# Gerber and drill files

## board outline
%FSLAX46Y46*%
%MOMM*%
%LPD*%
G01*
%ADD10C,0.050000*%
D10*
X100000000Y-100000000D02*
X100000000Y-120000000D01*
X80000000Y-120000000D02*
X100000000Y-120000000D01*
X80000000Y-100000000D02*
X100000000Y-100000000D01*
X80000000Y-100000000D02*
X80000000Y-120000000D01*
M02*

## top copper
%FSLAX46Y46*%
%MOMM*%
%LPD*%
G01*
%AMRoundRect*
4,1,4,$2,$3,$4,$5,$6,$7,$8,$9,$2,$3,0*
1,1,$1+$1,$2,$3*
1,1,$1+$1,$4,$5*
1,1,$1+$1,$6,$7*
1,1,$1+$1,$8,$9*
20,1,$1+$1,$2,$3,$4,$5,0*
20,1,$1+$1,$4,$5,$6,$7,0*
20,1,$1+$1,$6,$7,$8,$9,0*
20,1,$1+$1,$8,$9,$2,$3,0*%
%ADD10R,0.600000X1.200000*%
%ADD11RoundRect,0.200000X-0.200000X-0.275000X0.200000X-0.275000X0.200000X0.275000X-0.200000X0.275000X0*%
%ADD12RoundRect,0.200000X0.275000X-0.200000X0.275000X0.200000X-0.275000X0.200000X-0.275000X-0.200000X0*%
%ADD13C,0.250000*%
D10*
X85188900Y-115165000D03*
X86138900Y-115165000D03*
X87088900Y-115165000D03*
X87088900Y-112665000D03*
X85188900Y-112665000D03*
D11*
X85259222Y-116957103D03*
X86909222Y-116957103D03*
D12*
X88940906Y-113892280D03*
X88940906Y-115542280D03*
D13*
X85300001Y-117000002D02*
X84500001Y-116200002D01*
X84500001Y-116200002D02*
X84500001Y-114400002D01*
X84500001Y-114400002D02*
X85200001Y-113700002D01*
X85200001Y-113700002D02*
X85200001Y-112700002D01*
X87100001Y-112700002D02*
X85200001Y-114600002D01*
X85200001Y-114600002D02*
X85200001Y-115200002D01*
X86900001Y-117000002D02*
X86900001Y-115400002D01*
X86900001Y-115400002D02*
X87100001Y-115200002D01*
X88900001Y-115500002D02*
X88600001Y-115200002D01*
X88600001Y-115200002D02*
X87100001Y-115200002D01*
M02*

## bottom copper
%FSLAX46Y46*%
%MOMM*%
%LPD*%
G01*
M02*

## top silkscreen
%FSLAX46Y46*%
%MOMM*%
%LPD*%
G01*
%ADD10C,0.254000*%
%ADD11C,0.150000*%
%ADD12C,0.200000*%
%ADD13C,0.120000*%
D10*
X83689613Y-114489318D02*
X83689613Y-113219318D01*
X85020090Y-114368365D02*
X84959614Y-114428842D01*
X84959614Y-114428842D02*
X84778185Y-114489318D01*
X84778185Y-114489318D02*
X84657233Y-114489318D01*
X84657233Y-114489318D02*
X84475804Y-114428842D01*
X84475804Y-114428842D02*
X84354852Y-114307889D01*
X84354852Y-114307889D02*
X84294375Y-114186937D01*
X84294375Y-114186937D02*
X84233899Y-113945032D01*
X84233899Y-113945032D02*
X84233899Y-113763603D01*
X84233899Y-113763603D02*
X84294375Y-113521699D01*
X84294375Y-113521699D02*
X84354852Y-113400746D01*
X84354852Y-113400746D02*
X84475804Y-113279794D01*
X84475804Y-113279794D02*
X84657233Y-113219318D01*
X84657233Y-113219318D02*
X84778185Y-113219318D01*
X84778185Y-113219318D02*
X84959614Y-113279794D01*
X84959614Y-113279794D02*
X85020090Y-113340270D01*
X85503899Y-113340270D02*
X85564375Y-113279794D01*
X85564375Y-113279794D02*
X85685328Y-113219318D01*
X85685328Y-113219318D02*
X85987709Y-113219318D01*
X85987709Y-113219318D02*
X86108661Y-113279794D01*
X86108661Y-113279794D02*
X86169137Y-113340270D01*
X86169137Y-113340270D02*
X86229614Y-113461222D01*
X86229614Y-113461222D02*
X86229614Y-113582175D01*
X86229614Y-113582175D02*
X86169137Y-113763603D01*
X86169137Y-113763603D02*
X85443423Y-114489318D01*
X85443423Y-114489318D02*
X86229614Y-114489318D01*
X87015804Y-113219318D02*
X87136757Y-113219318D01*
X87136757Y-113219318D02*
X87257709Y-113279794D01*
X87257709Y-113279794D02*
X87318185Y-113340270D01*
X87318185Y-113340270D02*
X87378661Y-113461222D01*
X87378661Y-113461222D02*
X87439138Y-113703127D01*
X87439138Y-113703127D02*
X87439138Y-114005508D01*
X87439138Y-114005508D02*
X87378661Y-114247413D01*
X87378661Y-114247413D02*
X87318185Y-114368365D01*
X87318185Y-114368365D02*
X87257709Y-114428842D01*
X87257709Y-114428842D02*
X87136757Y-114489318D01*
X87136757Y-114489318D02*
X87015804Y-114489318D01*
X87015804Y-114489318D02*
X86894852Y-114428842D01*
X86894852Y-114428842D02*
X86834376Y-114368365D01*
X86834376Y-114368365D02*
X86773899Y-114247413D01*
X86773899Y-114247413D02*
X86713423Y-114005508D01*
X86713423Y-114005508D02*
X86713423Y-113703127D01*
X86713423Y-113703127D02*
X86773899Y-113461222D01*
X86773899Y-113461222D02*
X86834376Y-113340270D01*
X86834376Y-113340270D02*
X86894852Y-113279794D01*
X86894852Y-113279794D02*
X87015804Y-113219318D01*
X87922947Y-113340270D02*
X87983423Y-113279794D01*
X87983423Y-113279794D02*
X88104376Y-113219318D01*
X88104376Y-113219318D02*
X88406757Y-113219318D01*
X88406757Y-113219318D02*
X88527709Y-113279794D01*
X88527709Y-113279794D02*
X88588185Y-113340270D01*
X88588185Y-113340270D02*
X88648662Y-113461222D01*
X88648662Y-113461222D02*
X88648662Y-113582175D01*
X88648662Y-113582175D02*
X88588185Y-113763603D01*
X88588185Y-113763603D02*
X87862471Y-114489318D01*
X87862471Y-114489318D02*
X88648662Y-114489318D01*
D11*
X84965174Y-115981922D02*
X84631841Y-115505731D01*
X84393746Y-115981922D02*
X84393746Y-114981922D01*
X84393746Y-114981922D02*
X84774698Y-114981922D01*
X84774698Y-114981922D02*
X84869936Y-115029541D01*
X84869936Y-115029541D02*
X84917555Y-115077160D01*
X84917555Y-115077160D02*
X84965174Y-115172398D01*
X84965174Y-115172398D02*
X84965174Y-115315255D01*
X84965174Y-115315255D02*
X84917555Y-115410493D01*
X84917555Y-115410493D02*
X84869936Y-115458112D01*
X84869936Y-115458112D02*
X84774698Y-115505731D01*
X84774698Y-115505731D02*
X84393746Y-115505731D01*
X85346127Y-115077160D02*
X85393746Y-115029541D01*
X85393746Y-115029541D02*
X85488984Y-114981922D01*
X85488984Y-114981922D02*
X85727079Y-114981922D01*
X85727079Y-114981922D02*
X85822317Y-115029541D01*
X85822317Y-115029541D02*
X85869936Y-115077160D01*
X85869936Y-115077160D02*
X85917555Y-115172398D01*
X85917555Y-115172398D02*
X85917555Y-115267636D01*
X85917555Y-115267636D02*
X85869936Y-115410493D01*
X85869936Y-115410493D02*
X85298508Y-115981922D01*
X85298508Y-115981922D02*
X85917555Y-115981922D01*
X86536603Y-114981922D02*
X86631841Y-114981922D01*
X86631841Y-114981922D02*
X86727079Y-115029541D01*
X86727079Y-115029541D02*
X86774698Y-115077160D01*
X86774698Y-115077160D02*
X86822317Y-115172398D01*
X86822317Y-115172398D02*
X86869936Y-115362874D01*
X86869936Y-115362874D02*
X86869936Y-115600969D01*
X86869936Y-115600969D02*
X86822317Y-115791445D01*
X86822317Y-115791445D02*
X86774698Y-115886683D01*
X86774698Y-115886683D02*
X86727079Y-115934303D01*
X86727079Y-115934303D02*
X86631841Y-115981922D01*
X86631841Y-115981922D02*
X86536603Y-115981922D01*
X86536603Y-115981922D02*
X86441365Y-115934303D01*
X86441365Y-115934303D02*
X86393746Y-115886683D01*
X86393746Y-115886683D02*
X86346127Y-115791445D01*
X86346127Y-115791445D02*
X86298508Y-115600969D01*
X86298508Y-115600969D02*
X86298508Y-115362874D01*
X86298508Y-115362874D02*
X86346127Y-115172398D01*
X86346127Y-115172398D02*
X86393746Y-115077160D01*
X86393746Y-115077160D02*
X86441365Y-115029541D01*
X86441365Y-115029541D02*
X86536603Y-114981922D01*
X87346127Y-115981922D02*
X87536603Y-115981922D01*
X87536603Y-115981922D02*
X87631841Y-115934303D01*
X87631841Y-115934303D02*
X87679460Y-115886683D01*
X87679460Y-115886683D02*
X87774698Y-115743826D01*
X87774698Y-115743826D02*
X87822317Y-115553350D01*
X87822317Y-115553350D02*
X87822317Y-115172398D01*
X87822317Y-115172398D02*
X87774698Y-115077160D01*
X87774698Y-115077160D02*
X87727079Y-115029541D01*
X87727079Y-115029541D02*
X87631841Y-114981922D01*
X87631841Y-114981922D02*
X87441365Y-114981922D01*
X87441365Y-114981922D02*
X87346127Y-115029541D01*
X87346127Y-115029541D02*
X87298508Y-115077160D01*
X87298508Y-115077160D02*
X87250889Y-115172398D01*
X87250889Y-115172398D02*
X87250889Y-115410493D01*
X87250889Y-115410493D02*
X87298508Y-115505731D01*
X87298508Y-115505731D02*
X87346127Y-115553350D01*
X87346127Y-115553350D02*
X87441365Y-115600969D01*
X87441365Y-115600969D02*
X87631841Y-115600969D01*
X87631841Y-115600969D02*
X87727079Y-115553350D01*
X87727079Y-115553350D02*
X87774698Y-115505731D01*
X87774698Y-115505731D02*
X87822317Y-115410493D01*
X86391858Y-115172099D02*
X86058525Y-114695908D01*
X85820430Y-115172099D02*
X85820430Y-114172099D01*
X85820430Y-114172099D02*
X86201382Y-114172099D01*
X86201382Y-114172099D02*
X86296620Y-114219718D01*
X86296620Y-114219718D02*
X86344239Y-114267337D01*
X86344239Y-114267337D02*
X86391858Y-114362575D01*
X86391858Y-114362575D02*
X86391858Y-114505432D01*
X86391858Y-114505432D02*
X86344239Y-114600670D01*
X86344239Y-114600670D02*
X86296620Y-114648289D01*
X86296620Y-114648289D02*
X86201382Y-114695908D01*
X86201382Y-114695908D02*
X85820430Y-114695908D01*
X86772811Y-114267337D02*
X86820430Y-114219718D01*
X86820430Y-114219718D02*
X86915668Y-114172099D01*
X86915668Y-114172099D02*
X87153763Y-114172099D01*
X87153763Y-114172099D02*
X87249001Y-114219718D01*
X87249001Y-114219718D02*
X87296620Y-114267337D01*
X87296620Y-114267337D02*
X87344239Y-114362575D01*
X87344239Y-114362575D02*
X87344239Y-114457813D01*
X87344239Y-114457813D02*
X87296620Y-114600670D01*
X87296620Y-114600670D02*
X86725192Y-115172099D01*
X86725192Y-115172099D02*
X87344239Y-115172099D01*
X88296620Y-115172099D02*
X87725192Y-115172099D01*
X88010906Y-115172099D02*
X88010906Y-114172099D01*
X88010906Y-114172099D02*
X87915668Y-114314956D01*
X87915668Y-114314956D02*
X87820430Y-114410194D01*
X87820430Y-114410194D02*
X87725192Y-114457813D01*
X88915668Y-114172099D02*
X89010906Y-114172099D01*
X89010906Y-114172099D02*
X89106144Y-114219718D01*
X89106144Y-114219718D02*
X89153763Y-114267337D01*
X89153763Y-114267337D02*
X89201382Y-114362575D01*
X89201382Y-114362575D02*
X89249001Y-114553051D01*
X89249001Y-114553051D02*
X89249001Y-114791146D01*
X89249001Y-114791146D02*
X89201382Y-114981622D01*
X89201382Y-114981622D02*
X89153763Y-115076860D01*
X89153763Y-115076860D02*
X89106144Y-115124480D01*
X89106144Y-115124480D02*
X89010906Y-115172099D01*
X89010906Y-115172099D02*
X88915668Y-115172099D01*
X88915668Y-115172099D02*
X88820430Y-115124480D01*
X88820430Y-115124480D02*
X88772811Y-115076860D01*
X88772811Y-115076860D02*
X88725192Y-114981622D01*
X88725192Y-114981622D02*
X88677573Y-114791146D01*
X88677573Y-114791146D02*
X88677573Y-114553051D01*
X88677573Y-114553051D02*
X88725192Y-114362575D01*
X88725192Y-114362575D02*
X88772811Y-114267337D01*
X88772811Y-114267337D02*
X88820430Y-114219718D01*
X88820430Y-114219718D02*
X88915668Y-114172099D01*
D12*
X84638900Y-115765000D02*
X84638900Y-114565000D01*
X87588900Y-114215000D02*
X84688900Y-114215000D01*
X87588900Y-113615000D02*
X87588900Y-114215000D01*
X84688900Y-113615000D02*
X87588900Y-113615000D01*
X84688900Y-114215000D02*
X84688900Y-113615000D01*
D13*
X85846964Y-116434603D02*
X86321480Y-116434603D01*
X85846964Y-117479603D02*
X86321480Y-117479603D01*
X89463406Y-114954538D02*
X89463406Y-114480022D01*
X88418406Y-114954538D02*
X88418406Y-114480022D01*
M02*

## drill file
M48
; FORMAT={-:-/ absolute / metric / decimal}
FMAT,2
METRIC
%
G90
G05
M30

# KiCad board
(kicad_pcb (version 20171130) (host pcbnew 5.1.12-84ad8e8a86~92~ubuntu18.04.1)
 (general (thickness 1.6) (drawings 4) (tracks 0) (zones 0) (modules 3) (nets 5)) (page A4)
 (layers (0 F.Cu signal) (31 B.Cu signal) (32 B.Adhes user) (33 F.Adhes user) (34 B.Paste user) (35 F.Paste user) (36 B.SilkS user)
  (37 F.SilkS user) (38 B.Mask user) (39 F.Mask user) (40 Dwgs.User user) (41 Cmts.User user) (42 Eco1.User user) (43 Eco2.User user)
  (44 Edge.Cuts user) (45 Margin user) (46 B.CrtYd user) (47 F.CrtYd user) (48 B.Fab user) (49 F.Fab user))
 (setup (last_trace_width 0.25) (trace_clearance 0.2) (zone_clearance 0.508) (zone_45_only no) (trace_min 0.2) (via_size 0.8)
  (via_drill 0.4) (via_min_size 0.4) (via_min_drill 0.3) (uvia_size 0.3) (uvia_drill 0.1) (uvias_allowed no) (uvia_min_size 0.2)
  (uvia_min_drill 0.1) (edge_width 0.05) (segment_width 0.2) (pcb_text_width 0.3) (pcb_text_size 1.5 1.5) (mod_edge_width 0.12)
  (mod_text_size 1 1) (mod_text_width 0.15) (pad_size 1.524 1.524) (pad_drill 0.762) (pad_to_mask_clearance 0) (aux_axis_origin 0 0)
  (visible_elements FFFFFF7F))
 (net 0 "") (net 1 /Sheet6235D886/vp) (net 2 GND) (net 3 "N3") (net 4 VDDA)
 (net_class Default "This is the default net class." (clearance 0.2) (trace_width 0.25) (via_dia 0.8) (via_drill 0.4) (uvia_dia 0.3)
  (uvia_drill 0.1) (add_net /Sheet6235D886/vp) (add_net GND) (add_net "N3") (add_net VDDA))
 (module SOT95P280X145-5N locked (layer F.Cu) (at 86.138900 113.915000 90.000000)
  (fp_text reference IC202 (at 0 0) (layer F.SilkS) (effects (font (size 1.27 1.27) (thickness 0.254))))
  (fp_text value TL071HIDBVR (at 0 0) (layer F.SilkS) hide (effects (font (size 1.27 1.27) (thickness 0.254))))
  (fp_line (start -1.85 -1.5) (end -0.65 -1.5) (layer F.SilkS) (width 0.2))
  (fp_line (start -0.3 1.45) (end -0.3 -1.45) (layer F.SilkS) (width 0.2))
  (fp_line (start 0.3 1.45) (end -0.3 1.45) (layer F.SilkS) (width 0.2))
  (fp_line (start 0.3 -1.45) (end 0.3 1.45) (layer F.SilkS) (width 0.2))
  (fp_line (start -0.3 -1.45) (end 0.3 -1.45) (layer F.SilkS) (width 0.2))
  (pad 1 smd rect (at -1.25 -0.95 180.000000) (size 0.6 1.2) (layers F.Cu F.Mask F.Paste) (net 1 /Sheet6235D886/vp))
  (pad 2 smd rect (at -1.25 0 180.000000) (size 0.6 1.2) (layers F.Cu F.Mask F.Paste) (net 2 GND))
  (pad 3 smd rect (at -1.25 0.95 180.000000) (size 0.6 1.2) (layers F.Cu F.Mask F.Paste) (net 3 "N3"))
  (pad 4 smd rect (at 1.25 0.95 180.000000) (size 0.6 1.2) (layers F.Cu F.Mask F.Paste) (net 1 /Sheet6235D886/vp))
  (pad 5 smd rect (at 1.25 -0.95 180.000000) (size 0.6 1.2) (layers F.Cu F.Mask F.Paste) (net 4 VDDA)))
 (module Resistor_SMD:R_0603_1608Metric (layer F.Cu) (at 86.084222 116.957103)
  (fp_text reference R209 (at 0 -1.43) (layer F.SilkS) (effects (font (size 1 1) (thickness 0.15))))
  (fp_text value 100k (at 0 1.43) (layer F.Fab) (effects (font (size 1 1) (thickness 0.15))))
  (fp_line (start -0.237258 -0.5225) (end 0.237258 -0.5225) (layer F.SilkS) (width 0.12))
  (fp_line (start -0.237258 0.5225) (end 0.237258 0.5225) (layer F.SilkS) (width 0.12))
  (pad 1 smd roundrect (at -0.825 0) (size 0.8 0.95) (layers F.Cu F.Mask F.Paste) (roundrect_rratio 0.25) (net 4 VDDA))
  (pad 2 smd roundrect (at 0.825 0) (size 0.8 0.95) (layers F.Cu F.Mask F.Paste) (roundrect_rratio 0.25) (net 3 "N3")))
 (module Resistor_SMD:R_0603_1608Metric (layer F.Cu) (at 88.940906 114.717280 90.000000)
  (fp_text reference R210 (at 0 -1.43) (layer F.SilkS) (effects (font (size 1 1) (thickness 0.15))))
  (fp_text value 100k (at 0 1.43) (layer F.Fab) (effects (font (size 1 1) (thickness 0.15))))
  (fp_line (start -0.237258 0.5225) (end 0.237258 0.5225) (layer F.SilkS) (width 0.12))
  (fp_line (start -0.237258 -0.5225) (end 0.237258 -0.5225) (layer F.SilkS) (width 0.12))
  (pad 2 smd roundrect (at 0.825 0 90.000000) (size 0.8 0.95) (layers F.Cu F.Mask F.Paste) (roundrect_rratio 0.25) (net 2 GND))
  (pad 1 smd roundrect (at -0.825 0 90.000000) (size 0.8 0.95) (layers F.Cu F.Mask F.Paste) (roundrect_rratio 0.25) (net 3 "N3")))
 (gr_line (start 100 100) (end 100 120) (layer Edge.Cuts) (width 0.05))
 (gr_line (start 80 120) (end 100 120) (layer Edge.Cuts) (width 0.05))
 (gr_line (start 80 100) (end 100 100) (layer Edge.Cuts) (width 0.05))
 (gr_line (start 80 100) (end 80 120) (layer Edge.Cuts) (width 0.05))
 (segment (start 85.300001 117.000002) (end 84.500001 116.200002) (width 0.250000) (layer F.Cu) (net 4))
 (segment (start 84.500001 116.200002) (end 84.500001 114.400002) (width 0.250000) (layer F.Cu) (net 4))
 (segment (start 84.500001 114.400002) (end 85.200001 113.700002) (width 0.250000) (layer F.Cu) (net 4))
 (segment (start 85.200001 113.700002) (end 85.200001 112.700002) (width 0.250000) (layer F.Cu) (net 4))
 (segment (start 87.100001 112.700002) (end 85.200001 114.600002) (width 0.250000) (layer F.Cu) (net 1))
 (segment (start 85.200001 114.600002) (end 85.200001 115.200002) (width 0.250000) (layer F.Cu) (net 1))
 (segment (start 86.900001 117.000002) (end 86.900001 115.400002) (width 0.250000) (layer F.Cu) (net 3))
 (segment (start 86.900001 115.400002) (end 87.100001 115.200002) (width 0.250000) (layer F.Cu) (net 3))
 (segment (start 88.900001 115.500002) (end 88.600001 115.200002) (width 0.250000) (layer F.Cu) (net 3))
 (segment (start 88.600001 115.200002) (end 87.100001 115.200002) (width 0.250000) (layer F.Cu) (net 3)))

